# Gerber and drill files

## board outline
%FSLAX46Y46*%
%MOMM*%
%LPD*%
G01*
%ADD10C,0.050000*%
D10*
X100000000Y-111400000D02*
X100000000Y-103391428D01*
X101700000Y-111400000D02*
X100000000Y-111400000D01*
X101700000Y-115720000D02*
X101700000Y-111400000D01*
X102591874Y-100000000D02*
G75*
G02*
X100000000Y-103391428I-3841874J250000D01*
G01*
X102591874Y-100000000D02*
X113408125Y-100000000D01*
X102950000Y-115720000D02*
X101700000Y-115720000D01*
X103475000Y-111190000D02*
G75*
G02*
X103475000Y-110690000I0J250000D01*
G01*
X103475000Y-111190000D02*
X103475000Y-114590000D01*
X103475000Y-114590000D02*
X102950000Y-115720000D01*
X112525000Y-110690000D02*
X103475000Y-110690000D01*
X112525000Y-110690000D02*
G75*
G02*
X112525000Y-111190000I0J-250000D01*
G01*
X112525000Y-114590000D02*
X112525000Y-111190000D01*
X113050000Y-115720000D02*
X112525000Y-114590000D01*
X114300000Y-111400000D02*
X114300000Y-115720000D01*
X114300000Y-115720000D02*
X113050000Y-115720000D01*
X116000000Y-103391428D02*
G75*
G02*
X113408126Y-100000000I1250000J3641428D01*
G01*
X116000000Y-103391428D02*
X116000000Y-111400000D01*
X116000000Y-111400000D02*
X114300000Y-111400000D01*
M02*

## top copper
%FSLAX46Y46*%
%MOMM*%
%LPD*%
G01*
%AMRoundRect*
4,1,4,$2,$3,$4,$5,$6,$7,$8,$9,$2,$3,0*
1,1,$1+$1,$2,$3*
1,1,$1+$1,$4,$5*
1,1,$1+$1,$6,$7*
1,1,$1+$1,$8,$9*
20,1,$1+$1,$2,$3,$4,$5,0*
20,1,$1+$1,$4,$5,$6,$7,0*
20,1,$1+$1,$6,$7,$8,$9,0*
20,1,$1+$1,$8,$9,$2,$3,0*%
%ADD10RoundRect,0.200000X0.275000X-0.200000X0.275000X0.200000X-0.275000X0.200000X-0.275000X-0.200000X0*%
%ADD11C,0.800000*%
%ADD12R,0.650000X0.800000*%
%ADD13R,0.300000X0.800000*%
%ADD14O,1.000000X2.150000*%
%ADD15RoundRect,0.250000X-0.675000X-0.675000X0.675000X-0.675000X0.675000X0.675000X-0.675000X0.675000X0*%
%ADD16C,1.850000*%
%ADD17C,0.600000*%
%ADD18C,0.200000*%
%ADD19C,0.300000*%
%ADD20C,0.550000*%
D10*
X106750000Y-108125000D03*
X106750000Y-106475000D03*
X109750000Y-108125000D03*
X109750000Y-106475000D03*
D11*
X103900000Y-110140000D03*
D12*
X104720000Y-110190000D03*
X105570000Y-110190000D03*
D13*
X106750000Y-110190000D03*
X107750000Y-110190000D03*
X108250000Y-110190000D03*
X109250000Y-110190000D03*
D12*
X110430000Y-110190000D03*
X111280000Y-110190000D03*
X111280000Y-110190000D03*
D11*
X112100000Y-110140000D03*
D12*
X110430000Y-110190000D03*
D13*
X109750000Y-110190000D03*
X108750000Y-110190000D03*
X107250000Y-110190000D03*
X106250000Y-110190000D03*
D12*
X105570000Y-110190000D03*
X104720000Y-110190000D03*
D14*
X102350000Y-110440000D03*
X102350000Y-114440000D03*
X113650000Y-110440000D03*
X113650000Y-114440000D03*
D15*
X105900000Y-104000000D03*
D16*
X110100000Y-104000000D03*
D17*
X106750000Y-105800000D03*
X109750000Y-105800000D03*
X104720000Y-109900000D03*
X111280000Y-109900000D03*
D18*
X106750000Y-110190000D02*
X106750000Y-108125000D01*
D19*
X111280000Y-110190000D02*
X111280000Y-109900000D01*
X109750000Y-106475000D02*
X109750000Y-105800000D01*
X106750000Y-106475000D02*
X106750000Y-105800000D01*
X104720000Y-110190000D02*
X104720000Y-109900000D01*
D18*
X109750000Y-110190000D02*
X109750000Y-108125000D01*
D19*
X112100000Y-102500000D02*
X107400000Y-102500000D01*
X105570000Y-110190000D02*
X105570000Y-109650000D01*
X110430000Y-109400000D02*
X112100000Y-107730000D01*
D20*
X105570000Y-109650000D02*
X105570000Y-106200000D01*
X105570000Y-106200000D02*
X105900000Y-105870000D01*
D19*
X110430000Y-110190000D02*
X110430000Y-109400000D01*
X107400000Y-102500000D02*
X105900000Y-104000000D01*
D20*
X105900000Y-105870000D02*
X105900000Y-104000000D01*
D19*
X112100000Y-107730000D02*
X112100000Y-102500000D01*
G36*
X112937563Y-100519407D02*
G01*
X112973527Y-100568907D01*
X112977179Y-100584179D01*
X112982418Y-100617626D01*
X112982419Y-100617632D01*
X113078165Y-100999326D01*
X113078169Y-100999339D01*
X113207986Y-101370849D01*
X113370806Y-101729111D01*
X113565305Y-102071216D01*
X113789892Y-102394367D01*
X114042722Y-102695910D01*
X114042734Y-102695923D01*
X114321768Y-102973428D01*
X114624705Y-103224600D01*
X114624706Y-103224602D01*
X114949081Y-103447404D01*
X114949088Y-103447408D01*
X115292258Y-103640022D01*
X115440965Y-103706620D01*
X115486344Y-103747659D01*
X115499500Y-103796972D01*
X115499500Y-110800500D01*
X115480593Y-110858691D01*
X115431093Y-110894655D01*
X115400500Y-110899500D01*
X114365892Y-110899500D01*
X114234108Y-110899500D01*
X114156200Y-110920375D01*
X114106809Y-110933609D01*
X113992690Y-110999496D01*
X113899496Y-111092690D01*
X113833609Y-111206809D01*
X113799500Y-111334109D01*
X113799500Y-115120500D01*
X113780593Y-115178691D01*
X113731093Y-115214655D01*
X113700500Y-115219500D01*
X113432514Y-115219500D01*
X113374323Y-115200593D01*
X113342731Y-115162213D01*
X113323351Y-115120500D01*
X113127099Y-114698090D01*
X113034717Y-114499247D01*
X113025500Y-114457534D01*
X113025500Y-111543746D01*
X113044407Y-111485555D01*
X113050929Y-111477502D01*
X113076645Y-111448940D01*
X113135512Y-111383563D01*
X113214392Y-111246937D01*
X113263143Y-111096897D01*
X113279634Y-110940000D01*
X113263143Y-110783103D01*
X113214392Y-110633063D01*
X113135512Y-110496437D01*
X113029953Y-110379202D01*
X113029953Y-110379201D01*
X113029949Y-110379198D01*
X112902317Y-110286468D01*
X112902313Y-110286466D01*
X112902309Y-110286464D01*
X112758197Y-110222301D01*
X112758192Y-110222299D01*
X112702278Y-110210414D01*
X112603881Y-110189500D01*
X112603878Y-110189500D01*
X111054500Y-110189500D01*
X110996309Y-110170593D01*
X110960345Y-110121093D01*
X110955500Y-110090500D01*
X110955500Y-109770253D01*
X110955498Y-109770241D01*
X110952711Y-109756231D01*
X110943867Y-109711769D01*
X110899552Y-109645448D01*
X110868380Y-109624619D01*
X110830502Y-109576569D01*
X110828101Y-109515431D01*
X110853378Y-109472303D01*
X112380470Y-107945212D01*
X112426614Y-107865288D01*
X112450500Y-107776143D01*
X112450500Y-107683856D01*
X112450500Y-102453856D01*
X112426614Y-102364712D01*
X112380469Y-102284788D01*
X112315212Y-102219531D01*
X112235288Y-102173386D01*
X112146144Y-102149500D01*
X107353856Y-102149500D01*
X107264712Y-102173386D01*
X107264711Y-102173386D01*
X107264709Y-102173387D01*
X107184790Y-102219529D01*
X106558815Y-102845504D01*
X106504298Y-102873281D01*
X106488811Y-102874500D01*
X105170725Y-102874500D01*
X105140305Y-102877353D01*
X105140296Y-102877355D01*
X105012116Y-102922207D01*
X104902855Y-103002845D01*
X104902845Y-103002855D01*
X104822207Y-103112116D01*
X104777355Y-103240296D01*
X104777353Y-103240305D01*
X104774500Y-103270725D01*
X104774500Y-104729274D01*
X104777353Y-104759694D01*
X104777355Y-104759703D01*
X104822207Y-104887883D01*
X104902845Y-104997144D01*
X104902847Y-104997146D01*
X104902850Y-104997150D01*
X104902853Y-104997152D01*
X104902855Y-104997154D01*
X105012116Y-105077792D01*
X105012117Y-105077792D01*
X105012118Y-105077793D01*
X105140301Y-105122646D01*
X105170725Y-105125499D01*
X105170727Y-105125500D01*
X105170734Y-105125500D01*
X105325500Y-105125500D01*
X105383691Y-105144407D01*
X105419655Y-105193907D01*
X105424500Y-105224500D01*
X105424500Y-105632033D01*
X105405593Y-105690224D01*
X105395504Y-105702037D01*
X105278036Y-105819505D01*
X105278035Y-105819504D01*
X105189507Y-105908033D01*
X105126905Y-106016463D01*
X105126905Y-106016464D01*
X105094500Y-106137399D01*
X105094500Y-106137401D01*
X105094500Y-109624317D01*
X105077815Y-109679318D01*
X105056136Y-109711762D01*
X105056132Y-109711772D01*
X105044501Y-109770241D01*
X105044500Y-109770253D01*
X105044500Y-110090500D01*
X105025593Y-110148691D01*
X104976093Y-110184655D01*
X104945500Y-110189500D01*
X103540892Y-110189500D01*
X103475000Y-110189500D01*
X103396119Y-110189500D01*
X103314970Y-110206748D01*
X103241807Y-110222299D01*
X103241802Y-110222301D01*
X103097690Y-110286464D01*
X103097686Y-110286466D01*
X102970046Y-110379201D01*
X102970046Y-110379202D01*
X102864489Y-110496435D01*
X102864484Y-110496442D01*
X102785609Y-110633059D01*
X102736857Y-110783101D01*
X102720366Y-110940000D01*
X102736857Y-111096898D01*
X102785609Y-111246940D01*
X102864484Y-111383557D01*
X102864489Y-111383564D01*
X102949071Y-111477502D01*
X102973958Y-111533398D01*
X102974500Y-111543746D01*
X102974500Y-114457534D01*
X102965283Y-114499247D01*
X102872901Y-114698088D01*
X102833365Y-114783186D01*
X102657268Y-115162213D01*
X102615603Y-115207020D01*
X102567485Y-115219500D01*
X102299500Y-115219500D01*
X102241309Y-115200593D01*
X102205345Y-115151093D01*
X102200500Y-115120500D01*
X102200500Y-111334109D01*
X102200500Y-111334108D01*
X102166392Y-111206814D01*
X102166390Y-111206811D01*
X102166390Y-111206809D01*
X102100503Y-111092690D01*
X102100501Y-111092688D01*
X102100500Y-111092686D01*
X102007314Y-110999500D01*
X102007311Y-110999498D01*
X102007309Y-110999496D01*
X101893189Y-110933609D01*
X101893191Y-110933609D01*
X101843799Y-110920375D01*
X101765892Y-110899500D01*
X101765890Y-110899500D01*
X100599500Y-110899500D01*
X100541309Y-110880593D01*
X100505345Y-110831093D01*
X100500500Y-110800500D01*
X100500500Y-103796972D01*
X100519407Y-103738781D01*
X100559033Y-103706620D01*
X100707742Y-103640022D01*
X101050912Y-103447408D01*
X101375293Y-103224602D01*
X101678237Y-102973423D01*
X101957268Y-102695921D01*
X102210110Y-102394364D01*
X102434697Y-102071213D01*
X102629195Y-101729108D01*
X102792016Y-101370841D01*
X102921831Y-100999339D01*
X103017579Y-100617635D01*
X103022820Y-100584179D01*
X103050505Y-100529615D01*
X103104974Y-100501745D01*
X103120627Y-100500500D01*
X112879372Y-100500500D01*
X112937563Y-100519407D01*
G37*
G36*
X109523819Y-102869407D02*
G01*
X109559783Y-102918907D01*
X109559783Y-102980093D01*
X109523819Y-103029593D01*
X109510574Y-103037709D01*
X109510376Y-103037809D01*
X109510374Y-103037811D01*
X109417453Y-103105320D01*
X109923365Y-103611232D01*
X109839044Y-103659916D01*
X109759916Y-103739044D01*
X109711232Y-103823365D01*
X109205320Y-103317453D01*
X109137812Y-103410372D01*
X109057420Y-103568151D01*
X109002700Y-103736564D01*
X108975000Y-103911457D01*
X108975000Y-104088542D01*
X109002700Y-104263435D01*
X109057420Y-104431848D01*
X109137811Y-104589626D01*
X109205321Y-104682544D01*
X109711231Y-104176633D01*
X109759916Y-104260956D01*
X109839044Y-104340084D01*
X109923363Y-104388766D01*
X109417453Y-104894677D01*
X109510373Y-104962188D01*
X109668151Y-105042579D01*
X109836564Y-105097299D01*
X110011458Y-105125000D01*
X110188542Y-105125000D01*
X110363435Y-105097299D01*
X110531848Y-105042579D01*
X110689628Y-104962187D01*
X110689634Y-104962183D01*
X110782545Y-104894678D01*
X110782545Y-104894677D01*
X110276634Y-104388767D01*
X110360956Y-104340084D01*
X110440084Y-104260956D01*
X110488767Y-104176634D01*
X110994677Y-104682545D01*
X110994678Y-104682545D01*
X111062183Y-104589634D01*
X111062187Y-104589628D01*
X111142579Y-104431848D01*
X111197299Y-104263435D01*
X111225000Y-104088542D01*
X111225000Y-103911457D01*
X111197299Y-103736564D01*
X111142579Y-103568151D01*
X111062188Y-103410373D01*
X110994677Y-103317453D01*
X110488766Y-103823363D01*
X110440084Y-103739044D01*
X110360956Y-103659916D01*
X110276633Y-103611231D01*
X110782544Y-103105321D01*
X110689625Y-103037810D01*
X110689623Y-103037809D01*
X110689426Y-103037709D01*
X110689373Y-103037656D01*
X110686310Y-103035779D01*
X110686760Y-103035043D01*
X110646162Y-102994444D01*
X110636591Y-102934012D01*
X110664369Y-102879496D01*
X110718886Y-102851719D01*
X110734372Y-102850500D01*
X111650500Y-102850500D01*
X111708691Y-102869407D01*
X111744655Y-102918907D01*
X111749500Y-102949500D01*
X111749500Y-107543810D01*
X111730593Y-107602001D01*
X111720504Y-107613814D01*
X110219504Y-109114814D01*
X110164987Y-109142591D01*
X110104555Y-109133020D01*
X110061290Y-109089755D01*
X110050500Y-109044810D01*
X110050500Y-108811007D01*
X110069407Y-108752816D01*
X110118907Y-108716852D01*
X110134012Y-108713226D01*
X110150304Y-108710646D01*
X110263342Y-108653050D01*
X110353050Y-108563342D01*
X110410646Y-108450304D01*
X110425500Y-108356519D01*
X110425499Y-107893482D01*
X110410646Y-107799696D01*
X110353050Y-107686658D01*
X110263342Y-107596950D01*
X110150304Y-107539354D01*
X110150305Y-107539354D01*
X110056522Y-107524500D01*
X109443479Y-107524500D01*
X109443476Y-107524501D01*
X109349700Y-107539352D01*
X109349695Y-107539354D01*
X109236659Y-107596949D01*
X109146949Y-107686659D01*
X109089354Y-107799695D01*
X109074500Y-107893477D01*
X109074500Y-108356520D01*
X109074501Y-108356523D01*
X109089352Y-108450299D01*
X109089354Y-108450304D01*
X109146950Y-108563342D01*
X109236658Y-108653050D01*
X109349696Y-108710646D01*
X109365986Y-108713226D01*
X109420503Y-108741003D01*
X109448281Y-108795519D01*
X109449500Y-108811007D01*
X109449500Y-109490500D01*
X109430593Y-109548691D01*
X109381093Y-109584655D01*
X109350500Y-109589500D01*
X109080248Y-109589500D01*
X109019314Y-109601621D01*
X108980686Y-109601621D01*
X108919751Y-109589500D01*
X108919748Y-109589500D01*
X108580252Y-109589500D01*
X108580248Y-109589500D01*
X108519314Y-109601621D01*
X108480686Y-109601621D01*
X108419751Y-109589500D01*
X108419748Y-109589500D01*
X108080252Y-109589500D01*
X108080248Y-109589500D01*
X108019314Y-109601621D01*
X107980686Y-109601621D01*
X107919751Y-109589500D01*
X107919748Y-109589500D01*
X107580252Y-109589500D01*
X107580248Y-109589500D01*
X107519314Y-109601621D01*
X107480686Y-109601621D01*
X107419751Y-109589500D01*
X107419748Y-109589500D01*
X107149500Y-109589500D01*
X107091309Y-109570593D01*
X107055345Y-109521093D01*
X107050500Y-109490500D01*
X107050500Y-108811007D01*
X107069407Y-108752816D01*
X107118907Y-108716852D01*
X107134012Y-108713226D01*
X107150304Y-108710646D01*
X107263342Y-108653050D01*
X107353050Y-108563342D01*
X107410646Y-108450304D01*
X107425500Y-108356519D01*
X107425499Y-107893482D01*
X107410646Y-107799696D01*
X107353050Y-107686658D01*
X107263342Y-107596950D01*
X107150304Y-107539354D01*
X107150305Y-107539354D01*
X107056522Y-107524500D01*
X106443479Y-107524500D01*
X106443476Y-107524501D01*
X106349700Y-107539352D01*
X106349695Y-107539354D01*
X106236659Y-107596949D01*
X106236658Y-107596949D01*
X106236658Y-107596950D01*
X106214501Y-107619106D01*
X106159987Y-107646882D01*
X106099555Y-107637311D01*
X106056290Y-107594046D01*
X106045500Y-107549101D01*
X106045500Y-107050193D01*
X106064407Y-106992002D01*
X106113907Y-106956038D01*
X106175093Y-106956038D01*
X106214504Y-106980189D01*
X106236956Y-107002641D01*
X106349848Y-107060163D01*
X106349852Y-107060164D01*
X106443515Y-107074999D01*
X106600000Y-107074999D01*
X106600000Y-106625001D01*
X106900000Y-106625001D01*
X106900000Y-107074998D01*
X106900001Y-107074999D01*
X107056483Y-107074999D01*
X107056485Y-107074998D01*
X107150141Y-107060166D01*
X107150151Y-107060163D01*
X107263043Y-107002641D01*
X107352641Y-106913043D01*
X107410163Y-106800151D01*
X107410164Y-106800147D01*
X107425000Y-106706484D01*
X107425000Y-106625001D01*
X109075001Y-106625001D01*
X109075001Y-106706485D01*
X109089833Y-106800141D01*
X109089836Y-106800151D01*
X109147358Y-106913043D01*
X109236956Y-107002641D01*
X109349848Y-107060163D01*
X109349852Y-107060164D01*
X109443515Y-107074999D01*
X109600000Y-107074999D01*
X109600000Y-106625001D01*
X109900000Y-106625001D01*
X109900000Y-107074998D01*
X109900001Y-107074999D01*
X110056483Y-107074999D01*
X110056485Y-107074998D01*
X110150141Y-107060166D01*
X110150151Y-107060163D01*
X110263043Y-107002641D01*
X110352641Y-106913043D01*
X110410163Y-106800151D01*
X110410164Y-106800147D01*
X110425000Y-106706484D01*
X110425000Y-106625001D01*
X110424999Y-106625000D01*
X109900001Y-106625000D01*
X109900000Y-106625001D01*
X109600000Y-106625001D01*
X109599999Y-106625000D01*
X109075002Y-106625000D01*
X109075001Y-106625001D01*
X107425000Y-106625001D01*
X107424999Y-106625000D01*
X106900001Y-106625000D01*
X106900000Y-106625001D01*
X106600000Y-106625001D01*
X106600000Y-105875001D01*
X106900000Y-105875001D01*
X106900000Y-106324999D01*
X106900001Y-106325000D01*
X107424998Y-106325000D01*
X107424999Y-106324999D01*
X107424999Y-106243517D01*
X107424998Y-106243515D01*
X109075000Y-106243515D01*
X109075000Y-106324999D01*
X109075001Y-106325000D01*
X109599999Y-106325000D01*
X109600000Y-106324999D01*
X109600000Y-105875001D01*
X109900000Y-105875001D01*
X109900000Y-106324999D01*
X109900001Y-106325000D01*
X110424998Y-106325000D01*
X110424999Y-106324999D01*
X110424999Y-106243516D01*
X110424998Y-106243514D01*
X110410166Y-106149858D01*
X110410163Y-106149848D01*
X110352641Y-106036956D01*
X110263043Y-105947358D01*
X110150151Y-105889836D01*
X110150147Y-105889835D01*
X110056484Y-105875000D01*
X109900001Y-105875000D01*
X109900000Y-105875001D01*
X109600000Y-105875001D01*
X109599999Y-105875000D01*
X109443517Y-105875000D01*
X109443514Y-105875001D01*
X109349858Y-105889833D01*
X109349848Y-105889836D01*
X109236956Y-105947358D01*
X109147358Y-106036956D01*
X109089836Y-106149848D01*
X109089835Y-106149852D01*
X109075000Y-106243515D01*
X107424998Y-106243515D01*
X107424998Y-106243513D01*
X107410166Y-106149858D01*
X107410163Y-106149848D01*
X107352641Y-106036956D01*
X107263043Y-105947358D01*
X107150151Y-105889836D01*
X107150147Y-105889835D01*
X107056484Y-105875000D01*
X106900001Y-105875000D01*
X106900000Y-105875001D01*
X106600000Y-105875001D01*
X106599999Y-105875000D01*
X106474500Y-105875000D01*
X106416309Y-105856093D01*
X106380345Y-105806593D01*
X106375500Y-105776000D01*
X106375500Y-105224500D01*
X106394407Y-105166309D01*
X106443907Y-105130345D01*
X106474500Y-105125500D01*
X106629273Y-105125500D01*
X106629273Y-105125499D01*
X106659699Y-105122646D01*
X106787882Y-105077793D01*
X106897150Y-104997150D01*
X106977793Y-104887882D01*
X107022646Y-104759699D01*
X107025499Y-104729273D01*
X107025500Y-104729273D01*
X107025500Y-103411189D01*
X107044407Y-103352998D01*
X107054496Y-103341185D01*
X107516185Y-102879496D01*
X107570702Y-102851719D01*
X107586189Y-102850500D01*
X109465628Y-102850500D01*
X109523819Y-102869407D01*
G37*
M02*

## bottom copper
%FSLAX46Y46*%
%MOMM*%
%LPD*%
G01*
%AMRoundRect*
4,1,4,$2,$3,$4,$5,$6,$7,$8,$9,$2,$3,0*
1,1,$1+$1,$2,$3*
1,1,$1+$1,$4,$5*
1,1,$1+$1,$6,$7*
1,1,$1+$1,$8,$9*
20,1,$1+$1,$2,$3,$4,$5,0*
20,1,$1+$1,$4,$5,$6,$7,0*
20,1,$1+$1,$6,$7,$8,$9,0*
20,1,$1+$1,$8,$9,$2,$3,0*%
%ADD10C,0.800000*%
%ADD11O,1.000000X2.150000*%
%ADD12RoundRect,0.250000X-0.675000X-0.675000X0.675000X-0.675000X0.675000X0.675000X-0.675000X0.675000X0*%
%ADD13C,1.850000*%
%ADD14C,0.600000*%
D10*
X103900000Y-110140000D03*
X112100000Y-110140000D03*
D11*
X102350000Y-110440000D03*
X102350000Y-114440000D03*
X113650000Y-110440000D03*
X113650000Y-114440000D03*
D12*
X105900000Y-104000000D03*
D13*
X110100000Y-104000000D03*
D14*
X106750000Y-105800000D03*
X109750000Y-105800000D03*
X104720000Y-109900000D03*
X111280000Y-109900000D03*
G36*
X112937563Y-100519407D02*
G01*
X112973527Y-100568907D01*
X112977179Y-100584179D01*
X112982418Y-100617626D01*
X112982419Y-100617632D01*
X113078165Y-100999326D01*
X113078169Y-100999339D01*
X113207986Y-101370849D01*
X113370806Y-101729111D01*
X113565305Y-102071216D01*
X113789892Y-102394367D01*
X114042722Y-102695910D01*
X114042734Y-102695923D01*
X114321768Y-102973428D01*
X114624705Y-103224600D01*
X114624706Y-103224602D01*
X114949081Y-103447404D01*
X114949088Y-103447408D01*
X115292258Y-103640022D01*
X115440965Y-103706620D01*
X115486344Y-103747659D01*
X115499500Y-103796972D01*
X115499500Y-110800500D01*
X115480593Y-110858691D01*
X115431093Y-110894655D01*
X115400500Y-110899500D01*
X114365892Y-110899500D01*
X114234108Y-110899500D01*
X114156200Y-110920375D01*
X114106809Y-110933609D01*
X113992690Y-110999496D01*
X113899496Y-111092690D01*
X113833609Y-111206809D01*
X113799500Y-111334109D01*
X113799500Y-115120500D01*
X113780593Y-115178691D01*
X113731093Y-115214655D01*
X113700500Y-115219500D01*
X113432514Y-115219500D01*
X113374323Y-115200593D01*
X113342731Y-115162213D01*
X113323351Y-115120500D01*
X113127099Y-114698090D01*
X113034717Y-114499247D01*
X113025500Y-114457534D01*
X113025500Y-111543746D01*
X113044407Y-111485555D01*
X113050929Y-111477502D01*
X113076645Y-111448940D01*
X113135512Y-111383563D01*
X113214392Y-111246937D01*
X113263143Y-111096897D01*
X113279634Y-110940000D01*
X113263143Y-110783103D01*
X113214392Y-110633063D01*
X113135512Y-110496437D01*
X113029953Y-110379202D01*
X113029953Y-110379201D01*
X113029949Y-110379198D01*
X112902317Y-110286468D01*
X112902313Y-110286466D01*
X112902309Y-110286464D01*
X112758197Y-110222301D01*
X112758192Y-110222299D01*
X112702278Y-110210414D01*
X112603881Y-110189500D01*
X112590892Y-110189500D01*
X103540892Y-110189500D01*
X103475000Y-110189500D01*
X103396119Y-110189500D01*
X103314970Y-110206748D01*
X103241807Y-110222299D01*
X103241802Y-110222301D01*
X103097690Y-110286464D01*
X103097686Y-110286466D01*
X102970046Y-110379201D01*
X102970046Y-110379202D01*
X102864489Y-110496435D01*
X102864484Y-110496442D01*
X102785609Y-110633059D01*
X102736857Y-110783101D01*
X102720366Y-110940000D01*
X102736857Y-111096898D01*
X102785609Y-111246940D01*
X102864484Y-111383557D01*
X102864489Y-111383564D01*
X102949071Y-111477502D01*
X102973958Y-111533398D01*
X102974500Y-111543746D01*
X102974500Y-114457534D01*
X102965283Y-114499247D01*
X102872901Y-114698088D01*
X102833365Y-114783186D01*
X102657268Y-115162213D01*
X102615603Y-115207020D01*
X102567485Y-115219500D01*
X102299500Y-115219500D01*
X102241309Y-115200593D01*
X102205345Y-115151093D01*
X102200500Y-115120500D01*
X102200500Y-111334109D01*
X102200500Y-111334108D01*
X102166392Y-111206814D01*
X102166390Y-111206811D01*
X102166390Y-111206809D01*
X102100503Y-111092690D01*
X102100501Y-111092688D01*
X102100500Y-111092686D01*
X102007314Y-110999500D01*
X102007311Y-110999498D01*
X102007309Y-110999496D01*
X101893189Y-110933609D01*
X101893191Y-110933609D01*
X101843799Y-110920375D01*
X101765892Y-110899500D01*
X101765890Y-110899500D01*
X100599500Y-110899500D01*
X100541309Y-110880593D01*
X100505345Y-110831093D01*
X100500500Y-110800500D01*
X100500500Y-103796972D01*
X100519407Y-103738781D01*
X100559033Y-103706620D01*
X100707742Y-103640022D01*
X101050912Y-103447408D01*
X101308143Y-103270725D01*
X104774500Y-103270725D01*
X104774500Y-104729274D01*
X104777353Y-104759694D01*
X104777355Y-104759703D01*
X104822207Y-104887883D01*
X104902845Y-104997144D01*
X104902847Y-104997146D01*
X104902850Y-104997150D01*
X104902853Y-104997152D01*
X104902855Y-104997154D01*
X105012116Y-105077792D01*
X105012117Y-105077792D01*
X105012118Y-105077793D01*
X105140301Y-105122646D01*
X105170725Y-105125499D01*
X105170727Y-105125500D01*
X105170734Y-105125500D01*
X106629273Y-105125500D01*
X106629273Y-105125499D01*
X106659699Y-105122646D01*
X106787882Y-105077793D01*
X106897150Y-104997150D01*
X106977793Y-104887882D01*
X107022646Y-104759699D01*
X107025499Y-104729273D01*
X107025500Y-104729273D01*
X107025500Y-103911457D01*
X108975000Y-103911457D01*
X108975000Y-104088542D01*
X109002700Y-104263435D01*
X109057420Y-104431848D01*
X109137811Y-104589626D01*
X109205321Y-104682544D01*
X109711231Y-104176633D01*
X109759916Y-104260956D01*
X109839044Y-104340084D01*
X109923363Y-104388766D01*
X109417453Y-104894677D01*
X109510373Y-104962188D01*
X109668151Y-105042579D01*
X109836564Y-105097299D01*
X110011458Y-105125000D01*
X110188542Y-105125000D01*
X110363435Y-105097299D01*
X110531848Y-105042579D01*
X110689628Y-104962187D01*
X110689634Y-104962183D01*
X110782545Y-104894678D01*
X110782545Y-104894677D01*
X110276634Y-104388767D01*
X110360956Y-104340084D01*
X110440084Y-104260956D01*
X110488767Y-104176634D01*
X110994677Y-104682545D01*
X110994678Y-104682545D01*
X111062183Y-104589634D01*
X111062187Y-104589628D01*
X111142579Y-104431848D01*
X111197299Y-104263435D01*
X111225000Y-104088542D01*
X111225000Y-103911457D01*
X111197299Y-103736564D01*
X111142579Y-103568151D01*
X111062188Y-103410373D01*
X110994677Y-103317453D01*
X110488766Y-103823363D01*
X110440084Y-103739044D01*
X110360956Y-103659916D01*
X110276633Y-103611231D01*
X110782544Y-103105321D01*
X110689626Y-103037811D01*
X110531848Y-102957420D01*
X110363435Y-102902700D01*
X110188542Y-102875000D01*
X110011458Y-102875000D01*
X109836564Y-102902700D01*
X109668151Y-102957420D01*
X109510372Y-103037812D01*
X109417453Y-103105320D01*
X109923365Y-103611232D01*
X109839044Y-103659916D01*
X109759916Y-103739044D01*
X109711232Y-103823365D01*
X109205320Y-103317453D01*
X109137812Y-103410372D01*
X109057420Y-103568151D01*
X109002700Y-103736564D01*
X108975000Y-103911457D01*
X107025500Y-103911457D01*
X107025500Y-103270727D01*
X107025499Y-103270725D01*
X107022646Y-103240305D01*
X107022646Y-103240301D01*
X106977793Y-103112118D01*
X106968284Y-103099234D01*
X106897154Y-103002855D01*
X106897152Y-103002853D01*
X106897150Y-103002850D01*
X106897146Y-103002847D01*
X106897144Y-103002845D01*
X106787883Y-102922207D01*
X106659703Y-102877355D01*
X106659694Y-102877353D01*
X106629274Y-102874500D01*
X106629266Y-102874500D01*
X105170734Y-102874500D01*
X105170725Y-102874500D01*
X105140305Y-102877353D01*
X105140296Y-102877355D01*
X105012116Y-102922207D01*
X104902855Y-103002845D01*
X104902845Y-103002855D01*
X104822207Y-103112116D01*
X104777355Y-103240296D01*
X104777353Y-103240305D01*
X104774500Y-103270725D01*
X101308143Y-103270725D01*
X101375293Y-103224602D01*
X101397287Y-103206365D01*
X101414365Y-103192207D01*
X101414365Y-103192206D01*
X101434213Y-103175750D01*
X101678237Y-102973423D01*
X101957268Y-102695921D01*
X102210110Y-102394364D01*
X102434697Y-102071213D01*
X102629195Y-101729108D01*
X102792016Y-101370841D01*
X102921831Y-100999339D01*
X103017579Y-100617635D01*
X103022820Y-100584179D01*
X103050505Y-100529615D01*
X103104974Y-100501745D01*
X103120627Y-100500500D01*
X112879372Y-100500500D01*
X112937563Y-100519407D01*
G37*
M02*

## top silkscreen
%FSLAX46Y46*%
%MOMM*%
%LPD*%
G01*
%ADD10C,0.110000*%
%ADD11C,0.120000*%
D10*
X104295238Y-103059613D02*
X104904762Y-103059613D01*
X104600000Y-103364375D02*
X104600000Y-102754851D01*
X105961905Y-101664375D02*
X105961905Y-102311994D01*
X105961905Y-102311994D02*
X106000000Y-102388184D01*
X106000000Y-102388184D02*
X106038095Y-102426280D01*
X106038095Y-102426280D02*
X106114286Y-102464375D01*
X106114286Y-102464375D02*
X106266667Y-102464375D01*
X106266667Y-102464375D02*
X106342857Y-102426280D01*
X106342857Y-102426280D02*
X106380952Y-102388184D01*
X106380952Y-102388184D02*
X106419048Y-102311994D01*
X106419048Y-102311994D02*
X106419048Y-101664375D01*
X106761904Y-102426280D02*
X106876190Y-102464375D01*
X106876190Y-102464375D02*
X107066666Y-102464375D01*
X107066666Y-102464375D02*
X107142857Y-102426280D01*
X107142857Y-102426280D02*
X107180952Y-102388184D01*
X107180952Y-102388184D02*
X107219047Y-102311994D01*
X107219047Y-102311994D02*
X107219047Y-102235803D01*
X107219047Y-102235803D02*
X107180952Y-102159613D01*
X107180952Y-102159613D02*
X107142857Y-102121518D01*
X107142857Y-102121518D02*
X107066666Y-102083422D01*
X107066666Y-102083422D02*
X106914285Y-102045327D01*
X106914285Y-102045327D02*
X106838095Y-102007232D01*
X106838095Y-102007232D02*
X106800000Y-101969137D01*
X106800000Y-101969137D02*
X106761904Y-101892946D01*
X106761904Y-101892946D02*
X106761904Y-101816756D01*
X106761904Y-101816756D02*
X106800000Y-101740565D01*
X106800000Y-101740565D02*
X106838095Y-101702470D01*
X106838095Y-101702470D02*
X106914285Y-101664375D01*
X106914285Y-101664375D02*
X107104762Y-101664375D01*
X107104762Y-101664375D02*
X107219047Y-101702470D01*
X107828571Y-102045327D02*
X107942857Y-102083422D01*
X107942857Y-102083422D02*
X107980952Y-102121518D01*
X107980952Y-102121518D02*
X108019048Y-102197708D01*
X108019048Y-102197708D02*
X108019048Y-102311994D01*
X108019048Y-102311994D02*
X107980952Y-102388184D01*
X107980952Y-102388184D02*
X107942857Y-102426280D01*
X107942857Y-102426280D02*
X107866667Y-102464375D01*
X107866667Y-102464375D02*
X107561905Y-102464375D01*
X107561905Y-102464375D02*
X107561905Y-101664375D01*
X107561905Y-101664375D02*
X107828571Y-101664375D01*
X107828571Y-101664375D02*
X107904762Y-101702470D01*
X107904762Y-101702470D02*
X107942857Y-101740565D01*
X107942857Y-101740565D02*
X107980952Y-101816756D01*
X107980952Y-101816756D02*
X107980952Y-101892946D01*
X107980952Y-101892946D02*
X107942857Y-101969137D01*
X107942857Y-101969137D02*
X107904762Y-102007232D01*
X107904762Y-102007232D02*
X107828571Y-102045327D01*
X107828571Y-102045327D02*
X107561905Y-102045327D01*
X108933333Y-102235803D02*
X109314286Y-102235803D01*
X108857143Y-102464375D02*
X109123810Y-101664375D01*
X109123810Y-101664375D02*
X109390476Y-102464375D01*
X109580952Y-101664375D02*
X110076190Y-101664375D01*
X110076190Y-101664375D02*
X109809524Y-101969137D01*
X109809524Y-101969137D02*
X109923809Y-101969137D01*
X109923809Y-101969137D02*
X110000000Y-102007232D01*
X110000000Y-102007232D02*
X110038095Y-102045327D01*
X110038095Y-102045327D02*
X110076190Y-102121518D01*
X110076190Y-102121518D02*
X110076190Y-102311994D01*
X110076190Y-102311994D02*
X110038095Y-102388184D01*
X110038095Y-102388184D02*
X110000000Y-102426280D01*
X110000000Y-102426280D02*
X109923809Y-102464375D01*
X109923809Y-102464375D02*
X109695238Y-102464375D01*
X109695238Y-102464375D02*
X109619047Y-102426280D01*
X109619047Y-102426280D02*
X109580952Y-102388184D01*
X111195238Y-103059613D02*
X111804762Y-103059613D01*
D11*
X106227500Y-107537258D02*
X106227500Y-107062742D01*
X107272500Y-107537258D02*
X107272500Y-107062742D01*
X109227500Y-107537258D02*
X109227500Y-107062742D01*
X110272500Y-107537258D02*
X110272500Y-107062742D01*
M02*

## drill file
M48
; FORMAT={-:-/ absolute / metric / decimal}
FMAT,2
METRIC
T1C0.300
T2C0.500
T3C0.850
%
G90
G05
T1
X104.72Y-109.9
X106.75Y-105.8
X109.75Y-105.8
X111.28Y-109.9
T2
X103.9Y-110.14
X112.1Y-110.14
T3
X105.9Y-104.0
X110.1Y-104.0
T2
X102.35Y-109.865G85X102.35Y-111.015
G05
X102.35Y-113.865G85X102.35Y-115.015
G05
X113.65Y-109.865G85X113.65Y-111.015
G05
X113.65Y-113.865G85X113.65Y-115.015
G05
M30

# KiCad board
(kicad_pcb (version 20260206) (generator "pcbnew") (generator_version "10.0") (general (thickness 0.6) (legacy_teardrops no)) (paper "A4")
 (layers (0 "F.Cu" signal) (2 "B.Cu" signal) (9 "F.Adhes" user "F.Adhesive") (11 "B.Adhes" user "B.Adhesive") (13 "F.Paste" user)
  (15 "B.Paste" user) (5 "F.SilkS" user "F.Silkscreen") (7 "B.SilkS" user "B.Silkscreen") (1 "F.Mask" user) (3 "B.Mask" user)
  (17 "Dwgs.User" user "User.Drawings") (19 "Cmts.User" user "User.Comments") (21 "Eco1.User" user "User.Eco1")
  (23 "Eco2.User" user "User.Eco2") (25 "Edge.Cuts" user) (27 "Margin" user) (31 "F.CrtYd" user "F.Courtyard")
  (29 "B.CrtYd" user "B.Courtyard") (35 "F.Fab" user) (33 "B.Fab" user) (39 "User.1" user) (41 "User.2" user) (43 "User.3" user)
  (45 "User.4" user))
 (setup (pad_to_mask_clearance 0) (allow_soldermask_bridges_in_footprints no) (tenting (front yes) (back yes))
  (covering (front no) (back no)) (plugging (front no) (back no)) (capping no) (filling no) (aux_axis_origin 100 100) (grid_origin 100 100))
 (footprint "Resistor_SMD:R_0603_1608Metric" (layer "F.Cu") (at 106.75 107.3 90)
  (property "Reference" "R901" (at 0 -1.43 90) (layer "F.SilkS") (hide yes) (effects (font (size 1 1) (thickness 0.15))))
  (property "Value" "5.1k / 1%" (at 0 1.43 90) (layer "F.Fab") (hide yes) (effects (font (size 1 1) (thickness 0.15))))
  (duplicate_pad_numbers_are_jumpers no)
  (fp_line (start -0.237258 -0.5225) (end 0.237258 -0.5225) (stroke (width 0.12) (type solid)) (layer "F.SilkS"))
  (fp_line (start -0.237258 0.5225) (end 0.237258 0.5225) (stroke (width 0.12) (type solid)) (layer "F.SilkS"))
  (pad "1" smd roundrect (at -0.825 0 90) (size 0.8 0.95) (layers "F.Cu" "F.Mask" "F.Paste") (roundrect_rratio 0.25) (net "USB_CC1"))
  (pad "2" smd roundrect (at 0.825 0 90) (size 0.8 0.95) (layers "F.Cu" "F.Mask" "F.Paste") (roundrect_rratio 0.25) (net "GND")))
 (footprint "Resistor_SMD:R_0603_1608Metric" (layer "F.Cu") (at 109.75 107.3 90)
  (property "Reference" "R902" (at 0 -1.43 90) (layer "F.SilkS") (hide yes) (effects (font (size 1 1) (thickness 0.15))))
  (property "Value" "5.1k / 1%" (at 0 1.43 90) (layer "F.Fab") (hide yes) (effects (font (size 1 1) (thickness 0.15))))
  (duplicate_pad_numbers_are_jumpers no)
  (fp_line (start -0.237258 -0.5225) (end 0.237258 -0.5225) (stroke (width 0.12) (type solid)) (layer "F.SilkS"))
  (fp_line (start -0.237258 0.5225) (end 0.237258 0.5225) (stroke (width 0.12) (type solid)) (layer "F.SilkS"))
  (pad "1" smd roundrect (at -0.825 0 90) (size 0.8 0.95) (layers "F.Cu" "F.Mask" "F.Paste") (roundrect_rratio 0.25) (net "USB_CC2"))
  (pad "2" smd roundrect (at 0.825 0 90) (size 0.8 0.95) (layers "F.Cu" "F.Mask" "F.Paste") (roundrect_rratio 0.25) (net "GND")))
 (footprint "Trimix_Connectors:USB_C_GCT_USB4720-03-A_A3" (layer "F.Cu") (at 108 110.14)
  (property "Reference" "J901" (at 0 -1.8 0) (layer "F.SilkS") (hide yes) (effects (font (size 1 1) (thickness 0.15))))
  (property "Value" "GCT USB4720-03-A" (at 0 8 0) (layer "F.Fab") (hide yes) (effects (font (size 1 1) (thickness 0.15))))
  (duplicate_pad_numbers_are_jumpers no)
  (pad "A1" thru_hole circle (at -4.1 0) (size 0.8 0.8) (drill 0.5) (layers "*.Cu" "*.Mask") (remove_unused_layers no) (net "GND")
   (zone_connect 2))
  (pad "A1" smd rect (at -3.28 0.05) (size 0.65 0.8) (layers "F.Cu" "F.Mask" "F.Paste") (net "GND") (zone_connect 2))
  (pad "A4" smd rect (at -2.43 0.05) (size 0.65 0.8) (layers "F.Cu" "F.Mask" "F.Paste") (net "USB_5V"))
  (pad "A5" smd rect (at -1.25 0.05) (size 0.3 0.8) (layers "F.Cu" "F.Mask" "F.Paste") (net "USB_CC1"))
  (pad "A6" smd rect (at -0.25 0.05) (size 0.3 0.8) (layers "F.Cu" "F.Mask" "F.Paste") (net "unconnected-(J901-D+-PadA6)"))
  (pad "A7" smd rect (at 0.25 0.05) (size 0.3 0.8) (layers "F.Cu" "F.Mask" "F.Paste") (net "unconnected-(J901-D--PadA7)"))
  (pad "A8" smd rect (at 1.25 0.05) (size 0.3 0.8) (layers "F.Cu" "F.Mask" "F.Paste") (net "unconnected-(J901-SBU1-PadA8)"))
  (pad "A9" smd rect (at 2.43 0.05) (size 0.65 0.8) (layers "F.Cu" "F.Mask" "F.Paste") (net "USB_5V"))
  (pad "A12" smd rect (at 3.28 0.05) (size 0.65 0.8) (layers "F.Cu" "F.Mask" "F.Paste") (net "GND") (zone_connect 2))
  (pad "B1" smd rect (at 3.28 0.05) (size 0.65 0.8) (layers "F.Cu" "F.Mask" "F.Paste") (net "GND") (zone_connect 2))
  (pad "B1" thru_hole circle (at 4.1 0) (size 0.8 0.8) (drill 0.5) (layers "*.Cu" "*.Mask") (remove_unused_layers no) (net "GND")
   (zone_connect 2))
  (pad "B4" smd rect (at 2.43 0.05) (size 0.65 0.8) (layers "F.Cu" "F.Mask" "F.Paste") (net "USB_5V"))
  (pad "B5" smd rect (at 1.75 0.05) (size 0.3 0.8) (layers "F.Cu" "F.Mask" "F.Paste") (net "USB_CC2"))
  (pad "B6" smd rect (at 0.75 0.05) (size 0.3 0.8) (layers "F.Cu" "F.Mask" "F.Paste") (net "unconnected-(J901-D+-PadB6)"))
  (pad "B7" smd rect (at -0.75 0.05) (size 0.3 0.8) (layers "F.Cu" "F.Mask" "F.Paste") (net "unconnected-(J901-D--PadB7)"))
  (pad "B8" smd rect (at -1.75 0.05) (size 0.3 0.8) (layers "F.Cu" "F.Mask" "F.Paste") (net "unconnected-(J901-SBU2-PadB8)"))
  (pad "B9" smd rect (at -2.43 0.05) (size 0.65 0.8) (layers "F.Cu" "F.Mask" "F.Paste") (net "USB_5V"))
  (pad "B12" smd rect (at -3.28 0.05) (size 0.65 0.8) (layers "F.Cu" "F.Mask" "F.Paste") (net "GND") (zone_connect 2))
  (pad "SH" thru_hole oval (at -5.65 0.3) (size 1 2.15) (drill oval 0.5 1.65) (layers "*.Cu" "*.Mask") (remove_unused_layers no) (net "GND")
   (zone_connect 2))
  (pad "SH" thru_hole oval (at -5.65 4.3) (size 1 2.15) (drill oval 0.5 1.65) (layers "*.Cu" "*.Mask") (remove_unused_layers no) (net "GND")
   (zone_connect 2))
  (pad "SH" thru_hole oval (at 5.65 0.3) (size 1 2.15) (drill oval 0.5 1.65) (layers "*.Cu" "*.Mask") (remove_unused_layers no) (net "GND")
   (zone_connect 2))
  (pad "SH" thru_hole oval (at 5.65 4.3) (size 1 2.15) (drill oval 0.5 1.65) (layers "*.Cu" "*.Mask") (remove_unused_layers no) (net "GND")
   (zone_connect 2)))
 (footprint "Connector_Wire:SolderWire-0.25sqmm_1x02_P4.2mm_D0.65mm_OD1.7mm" (layer "F.Cu") (at 105.9 104)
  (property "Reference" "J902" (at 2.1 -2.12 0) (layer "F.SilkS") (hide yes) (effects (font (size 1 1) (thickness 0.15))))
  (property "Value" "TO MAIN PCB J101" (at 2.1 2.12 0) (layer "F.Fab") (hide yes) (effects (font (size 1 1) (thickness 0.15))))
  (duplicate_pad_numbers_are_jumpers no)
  (pad "1" thru_hole roundrect (at 0 0) (size 1.85 1.85) (drill 0.85) (layers "*.Cu" "*.Mask") (remove_unused_layers no)
   (roundrect_rratio 0.135135) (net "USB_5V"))
  (pad "2" thru_hole circle (at 4.2 0) (size 1.85 1.85) (drill 0.85) (layers "*.Cu" "*.Mask") (remove_unused_layers no) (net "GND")))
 (gr_line (start 100 111.4) (end 100 103.391428) (stroke (width 0.05) (type default)) (layer "Edge.Cuts"))
 (gr_line (start 101.7 111.4) (end 100 111.4) (stroke (width 0.05) (type default)) (layer "Edge.Cuts"))
 (gr_line (start 101.7 115.72) (end 101.7 111.4) (stroke (width 0.05) (type default)) (layer "Edge.Cuts"))
 (gr_arc (start 102.591874 100) (mid 101.808961 102.087789) (end 100 103.391428) (stroke (width 0.05) (type default)) (layer "Edge.Cuts"))
 (gr_line (start 102.591874 100) (end 113.408125 100) (stroke (width 0.05) (type default)) (layer "Edge.Cuts"))
 (gr_line (start 102.95 115.72) (end 101.7 115.72) (stroke (width 0.05) (type default)) (layer "Edge.Cuts"))
 (gr_arc (start 103.475 111.19) (mid 103.225 110.94) (end 103.475 110.69) (stroke (width 0.05) (type default)) (layer "Edge.Cuts"))
 (gr_line (start 103.475 111.19) (end 103.475 114.59) (stroke (width 0.05) (type default)) (layer "Edge.Cuts"))
 (gr_line (start 103.475 114.59) (end 102.95 115.72) (stroke (width 0.05) (type default)) (layer "Edge.Cuts"))
 (gr_line (start 112.525 110.69) (end 103.475 110.69) (stroke (width 0.05) (type default)) (layer "Edge.Cuts"))
 (gr_arc (start 112.525 110.69) (mid 112.775 110.94) (end 112.525 111.19) (stroke (width 0.05) (type default)) (layer "Edge.Cuts"))
 (gr_line (start 112.525 114.59) (end 112.525 111.19) (stroke (width 0.05) (type default)) (layer "Edge.Cuts"))
 (gr_line (start 113.05 115.72) (end 112.525 114.59) (stroke (width 0.05) (type default)) (layer "Edge.Cuts"))
 (gr_line (start 114.3 111.4) (end 114.3 115.72) (stroke (width 0.05) (type default)) (layer "Edge.Cuts"))
 (gr_line (start 114.3 115.72) (end 113.05 115.72) (stroke (width 0.05) (type default)) (layer "Edge.Cuts"))
 (gr_arc (start 116 103.391428) (mid 114.191039 102.087789) (end 113.408125 100) (stroke (width 0.05) (type default)) (layer "Edge.Cuts"))
 (gr_line (start 116 103.391428) (end 116 111.4) (stroke (width 0.05) (type default)) (layer "Edge.Cuts"))
 (gr_line (start 116 111.4) (end 114.3 111.4) (stroke (width 0.05) (type default)) (layer "Edge.Cuts"))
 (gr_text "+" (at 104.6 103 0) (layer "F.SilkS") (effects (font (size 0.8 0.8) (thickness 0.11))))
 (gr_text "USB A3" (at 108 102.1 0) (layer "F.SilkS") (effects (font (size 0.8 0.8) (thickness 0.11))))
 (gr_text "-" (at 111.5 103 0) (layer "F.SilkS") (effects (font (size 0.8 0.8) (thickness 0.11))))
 (segment (start 106.75 110.19) (end 106.75 108.125) (width 0.2) (layer "F.Cu") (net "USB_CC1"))
 (segment (start 111.28 110.19) (end 111.28 109.9) (width 0.3) (layer "F.Cu") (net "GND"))
 (segment (start 109.75 106.475) (end 109.75 105.8) (width 0.3) (layer "F.Cu") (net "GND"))
 (segment (start 106.75 106.475) (end 106.75 105.8) (width 0.3) (layer "F.Cu") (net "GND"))
 (segment (start 104.72 110.19) (end 104.72 109.9) (width 0.3) (layer "F.Cu") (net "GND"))
 (via (at 106.75 105.8) (size 0.6) (drill 0.3) (layers "F.Cu" "B.Cu") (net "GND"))
 (via (at 109.75 105.8) (size 0.6) (drill 0.3) (layers "F.Cu" "B.Cu") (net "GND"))
 (via (at 104.72 109.9) (size 0.6) (drill 0.3) (layers "F.Cu" "B.Cu") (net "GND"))
 (via (at 111.28 109.9) (size 0.6) (drill 0.3) (layers "F.Cu" "B.Cu") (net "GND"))
 (segment (start 109.75 110.19) (end 109.75 108.125) (width 0.2) (layer "F.Cu") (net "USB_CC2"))
 (segment (start 112.1 102.5) (end 107.4 102.5) (width 0.3) (layer "F.Cu") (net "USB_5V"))
 (segment (start 105.57 110.19) (end 105.57 109.65) (width 0.3) (layer "F.Cu") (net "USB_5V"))
 (segment (start 110.43 109.4) (end 112.1 107.73) (width 0.3) (layer "F.Cu") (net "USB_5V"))
 (segment (start 105.57 109.65) (end 105.57 106.2) (width 0.55) (layer "F.Cu") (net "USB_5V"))
 (segment (start 105.57 106.2) (end 105.9 105.87) (width 0.55) (layer "F.Cu") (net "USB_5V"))
 (segment (start 110.43 110.19) (end 110.43 109.4) (width 0.3) (layer "F.Cu") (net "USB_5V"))
 (segment (start 107.4 102.5) (end 105.9 104) (width 0.3) (layer "F.Cu") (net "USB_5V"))
 (segment (start 105.9 105.87) (end 105.9 104) (width 0.55) (layer "F.Cu") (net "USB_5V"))
 (segment (start 112.1 107.73) (end 112.1 102.5) (width 0.3) (layer "F.Cu") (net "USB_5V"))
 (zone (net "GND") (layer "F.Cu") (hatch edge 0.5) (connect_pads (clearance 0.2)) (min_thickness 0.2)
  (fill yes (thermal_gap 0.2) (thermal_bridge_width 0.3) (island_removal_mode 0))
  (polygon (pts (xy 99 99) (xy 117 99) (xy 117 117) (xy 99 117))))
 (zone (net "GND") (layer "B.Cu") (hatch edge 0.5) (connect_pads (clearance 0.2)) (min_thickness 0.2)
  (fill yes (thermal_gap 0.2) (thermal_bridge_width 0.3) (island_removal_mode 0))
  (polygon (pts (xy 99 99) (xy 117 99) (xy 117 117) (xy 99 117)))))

